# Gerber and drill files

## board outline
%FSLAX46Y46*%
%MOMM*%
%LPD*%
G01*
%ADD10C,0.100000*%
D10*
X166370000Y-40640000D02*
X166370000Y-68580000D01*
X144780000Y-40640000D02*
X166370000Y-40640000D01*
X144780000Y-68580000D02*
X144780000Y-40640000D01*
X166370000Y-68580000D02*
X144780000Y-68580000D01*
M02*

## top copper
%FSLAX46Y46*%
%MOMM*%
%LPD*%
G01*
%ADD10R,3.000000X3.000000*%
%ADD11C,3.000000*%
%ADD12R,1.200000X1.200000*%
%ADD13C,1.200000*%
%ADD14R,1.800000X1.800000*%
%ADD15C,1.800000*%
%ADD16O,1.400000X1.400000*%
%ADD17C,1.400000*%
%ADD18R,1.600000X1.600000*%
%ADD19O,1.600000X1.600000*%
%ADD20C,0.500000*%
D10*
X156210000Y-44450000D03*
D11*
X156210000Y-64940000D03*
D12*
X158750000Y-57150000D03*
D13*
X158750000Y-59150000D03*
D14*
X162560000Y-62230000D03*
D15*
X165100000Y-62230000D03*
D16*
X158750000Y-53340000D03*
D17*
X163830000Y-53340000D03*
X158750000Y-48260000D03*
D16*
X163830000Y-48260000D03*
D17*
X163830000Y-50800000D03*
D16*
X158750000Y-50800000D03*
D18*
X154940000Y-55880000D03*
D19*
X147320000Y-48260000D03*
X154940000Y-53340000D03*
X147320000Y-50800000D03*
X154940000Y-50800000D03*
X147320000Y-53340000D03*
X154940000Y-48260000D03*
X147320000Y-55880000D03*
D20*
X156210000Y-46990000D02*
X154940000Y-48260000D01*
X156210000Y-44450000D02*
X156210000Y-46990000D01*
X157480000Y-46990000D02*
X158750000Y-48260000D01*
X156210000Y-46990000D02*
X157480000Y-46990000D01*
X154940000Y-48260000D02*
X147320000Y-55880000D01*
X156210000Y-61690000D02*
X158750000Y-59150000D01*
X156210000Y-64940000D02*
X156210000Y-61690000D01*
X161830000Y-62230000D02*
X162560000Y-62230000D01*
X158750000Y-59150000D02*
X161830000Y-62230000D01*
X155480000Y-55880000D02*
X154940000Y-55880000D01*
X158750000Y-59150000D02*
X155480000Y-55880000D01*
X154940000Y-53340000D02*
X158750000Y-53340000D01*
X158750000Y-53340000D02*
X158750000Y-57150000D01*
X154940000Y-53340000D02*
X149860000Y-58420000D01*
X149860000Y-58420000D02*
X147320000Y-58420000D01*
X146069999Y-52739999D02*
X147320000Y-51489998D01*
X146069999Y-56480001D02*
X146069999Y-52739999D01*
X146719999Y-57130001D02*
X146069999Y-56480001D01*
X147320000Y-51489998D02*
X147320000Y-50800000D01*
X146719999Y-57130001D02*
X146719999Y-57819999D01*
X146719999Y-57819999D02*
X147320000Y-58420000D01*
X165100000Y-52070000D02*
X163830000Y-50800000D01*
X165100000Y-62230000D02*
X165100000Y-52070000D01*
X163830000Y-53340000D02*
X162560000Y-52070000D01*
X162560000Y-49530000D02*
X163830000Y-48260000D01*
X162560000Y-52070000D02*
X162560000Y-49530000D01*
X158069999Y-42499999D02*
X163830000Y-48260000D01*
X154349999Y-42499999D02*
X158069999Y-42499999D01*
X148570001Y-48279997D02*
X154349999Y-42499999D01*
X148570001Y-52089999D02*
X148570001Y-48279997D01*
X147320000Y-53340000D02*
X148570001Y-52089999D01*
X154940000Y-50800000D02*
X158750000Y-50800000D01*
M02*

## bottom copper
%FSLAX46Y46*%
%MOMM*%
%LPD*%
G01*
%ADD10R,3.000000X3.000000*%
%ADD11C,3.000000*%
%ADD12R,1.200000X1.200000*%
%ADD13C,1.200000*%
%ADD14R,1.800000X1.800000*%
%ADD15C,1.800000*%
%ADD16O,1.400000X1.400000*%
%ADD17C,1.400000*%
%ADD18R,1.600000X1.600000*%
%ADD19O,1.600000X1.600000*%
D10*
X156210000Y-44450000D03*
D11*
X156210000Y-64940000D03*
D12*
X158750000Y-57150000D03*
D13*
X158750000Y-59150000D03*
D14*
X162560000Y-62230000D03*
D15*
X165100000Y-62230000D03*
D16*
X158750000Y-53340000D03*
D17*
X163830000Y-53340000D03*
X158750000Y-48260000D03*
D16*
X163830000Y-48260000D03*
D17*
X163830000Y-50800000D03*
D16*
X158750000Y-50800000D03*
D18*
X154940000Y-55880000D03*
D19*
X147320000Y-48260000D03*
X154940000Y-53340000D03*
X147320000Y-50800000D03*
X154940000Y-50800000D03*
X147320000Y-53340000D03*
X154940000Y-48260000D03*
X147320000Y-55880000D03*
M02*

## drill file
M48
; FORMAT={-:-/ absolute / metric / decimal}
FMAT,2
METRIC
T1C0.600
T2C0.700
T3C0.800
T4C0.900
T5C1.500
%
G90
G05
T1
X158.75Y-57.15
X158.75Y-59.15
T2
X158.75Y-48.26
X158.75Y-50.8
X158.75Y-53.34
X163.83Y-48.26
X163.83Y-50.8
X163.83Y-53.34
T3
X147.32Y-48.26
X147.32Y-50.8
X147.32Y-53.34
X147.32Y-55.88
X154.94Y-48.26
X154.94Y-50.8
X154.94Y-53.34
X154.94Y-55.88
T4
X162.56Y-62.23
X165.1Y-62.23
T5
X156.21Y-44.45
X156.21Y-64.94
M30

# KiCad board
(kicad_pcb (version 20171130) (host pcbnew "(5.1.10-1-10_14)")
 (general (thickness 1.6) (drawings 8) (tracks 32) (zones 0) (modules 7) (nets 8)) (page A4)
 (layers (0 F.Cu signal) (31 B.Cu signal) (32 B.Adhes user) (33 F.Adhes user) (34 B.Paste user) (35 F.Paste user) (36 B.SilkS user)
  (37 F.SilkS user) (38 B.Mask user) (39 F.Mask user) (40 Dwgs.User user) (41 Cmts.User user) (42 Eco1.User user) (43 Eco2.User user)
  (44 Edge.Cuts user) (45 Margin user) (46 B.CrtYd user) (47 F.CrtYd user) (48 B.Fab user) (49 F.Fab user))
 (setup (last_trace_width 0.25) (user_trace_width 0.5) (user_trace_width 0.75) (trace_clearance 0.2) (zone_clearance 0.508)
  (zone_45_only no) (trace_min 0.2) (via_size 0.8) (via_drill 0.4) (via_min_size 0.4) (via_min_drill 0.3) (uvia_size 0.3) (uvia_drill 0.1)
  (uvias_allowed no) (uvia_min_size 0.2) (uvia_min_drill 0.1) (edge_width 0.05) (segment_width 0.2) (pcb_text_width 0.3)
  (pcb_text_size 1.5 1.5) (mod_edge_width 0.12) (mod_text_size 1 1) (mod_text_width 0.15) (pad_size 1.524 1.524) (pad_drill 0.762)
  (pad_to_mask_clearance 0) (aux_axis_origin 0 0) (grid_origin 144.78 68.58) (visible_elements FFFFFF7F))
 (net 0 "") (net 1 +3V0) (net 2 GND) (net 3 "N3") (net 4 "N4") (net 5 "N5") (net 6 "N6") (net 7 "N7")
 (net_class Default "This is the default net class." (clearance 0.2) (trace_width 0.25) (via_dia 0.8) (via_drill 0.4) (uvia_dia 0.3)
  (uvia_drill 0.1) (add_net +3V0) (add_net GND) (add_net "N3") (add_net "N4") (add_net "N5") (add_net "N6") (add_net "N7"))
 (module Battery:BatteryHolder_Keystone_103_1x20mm (layer B.Cu) (at 156.21 44.45 270)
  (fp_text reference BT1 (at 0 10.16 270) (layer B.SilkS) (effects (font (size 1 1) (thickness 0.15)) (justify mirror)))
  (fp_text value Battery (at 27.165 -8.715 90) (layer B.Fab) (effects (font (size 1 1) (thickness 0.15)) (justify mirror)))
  (pad 1 thru_hole rect (at 0 0 270) (size 3 3) (drill 1.5) (layers *.Cu *.Mask) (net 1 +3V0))
  (pad 2 thru_hole circle (at 20.49 0 270) (size 3 3) (drill 1.5) (layers *.Cu *.Mask) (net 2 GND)))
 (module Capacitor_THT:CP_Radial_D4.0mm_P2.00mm (layer F.Cu) (at 158.75 57.15 270)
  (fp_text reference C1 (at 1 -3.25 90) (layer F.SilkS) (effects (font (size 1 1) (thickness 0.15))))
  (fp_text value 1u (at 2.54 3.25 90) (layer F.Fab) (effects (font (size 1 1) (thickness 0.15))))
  (pad 1 thru_hole rect (at 0 0 270) (size 1.2 1.2) (drill 0.6) (layers *.Cu *.Mask) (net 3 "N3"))
  (pad 2 thru_hole circle (at 2 0 270) (size 1.2 1.2) (drill 0.6) (layers *.Cu *.Mask) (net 2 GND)))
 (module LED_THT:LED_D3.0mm (layer F.Cu) (at 162.56 62.23)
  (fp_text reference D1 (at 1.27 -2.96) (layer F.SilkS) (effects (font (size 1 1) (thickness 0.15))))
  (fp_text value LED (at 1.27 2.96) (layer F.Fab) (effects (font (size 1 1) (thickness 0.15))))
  (pad 1 thru_hole rect (at 0 0) (size 1.8 1.8) (drill 0.9) (layers *.Cu *.Mask) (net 2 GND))
  (pad 2 thru_hole circle (at 2.54 0) (size 1.8 1.8) (drill 0.9) (layers *.Cu *.Mask) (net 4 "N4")))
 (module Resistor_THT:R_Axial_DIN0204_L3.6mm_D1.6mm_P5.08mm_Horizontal (layer F.Cu) (at 163.83 53.34 180)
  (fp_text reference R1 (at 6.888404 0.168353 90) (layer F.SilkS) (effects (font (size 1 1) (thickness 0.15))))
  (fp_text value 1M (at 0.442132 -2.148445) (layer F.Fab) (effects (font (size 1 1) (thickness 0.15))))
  (pad 2 thru_hole oval (at 5.08 0 180) (size 1.4 1.4) (drill 0.7) (layers *.Cu *.Mask) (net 3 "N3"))
  (pad 1 thru_hole circle (at 0 0 180) (size 1.4 1.4) (drill 0.7) (layers *.Cu *.Mask) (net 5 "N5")))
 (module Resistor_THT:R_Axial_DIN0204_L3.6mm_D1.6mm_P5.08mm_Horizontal (layer F.Cu) (at 158.75 48.26)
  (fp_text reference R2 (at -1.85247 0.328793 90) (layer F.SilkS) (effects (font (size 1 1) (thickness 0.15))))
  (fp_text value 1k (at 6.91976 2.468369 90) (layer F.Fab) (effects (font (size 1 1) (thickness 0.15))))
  (pad 1 thru_hole circle (at 0 0) (size 1.4 1.4) (drill 0.7) (layers *.Cu *.Mask) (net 1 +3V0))
  (pad 2 thru_hole oval (at 5.08 0) (size 1.4 1.4) (drill 0.7) (layers *.Cu *.Mask) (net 5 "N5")))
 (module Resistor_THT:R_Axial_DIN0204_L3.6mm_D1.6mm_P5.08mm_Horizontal (layer F.Cu) (at 163.83 50.8 180)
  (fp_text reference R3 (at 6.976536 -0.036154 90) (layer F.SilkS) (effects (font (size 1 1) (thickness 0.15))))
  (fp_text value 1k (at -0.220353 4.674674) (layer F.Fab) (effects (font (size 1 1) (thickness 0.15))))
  (pad 1 thru_hole circle (at 0 0 180) (size 1.4 1.4) (drill 0.7) (layers *.Cu *.Mask) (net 4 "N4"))
  (pad 2 thru_hole oval (at 5.08 0 180) (size 1.4 1.4) (drill 0.7) (layers *.Cu *.Mask) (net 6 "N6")))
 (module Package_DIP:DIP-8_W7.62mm (layer F.Cu) (at 154.94 55.88 180)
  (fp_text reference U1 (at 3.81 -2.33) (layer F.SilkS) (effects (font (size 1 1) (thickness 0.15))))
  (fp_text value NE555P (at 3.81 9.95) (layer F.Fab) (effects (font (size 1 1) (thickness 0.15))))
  (pad 1 thru_hole rect (at 0 0 180) (size 1.6 1.6) (drill 0.8) (layers *.Cu *.Mask) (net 2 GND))
  (pad 5 thru_hole oval (at 7.62 7.62 180) (size 1.6 1.6) (drill 0.8) (layers *.Cu *.Mask) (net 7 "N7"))
  (pad 2 thru_hole oval (at 0 2.54 180) (size 1.6 1.6) (drill 0.8) (layers *.Cu *.Mask) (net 3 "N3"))
  (pad 6 thru_hole oval (at 7.62 5.08 180) (size 1.6 1.6) (drill 0.8) (layers *.Cu *.Mask) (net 3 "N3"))
  (pad 3 thru_hole oval (at 0 5.08 180) (size 1.6 1.6) (drill 0.8) (layers *.Cu *.Mask) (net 6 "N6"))
  (pad 7 thru_hole oval (at 7.62 2.54 180) (size 1.6 1.6) (drill 0.8) (layers *.Cu *.Mask) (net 5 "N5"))
  (pad 4 thru_hole oval (at 0 7.62 180) (size 1.6 1.6) (drill 0.8) (layers *.Cu *.Mask) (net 1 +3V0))
  (pad 8 thru_hole oval (at 7.62 0 180) (size 1.6 1.6) (drill 0.8) (layers *.Cu *.Mask) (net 1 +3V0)))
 (gr_line (start 166.37 40.64) (end 166.37 68.58) (layer Edge.Cuts) (width 0.1))
 (gr_line (start 144.78 40.64) (end 166.37 40.64) (layer Edge.Cuts) (width 0.1))
 (gr_line (start 144.78 68.58) (end 144.78 40.64) (layer Edge.Cuts) (width 0.1))
 (gr_line (start 166.37 68.58) (end 144.78 68.58) (layer Edge.Cuts) (width 0.1))
 (segment (start 156.21 46.99) (end 154.94 48.26) (width 0.5) (layer F.Cu) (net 1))
 (segment (start 156.21 44.45) (end 156.21 46.99) (width 0.5) (layer F.Cu) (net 1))
 (segment (start 157.48 46.99) (end 158.75 48.26) (width 0.5) (layer F.Cu) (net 1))
 (segment (start 156.21 46.99) (end 157.48 46.99) (width 0.5) (layer F.Cu) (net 1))
 (segment (start 154.94 48.26) (end 147.32 55.88) (width 0.5) (layer F.Cu) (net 1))
 (segment (start 156.21 61.69) (end 158.75 59.15) (width 0.5) (layer F.Cu) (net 2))
 (segment (start 156.21 64.94) (end 156.21 61.69) (width 0.5) (layer F.Cu) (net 2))
 (segment (start 161.83 62.23) (end 162.56 62.23) (width 0.5) (layer F.Cu) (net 2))
 (segment (start 158.75 59.15) (end 161.83 62.23) (width 0.5) (layer F.Cu) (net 2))
 (segment (start 155.48 55.88) (end 154.94 55.88) (width 0.5) (layer F.Cu) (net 2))
 (segment (start 158.75 59.15) (end 155.48 55.88) (width 0.5) (layer F.Cu) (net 2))
 (segment (start 154.94 53.34) (end 158.75 53.34) (width 0.5) (layer F.Cu) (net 3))
 (segment (start 158.75 53.34) (end 158.75 57.15) (width 0.5) (layer F.Cu) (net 3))
 (segment (start 154.94 53.34) (end 149.86 58.42) (width 0.5) (layer F.Cu) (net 3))
 (segment (start 149.86 58.42) (end 147.32 58.42) (width 0.5) (layer F.Cu) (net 3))
 (segment (start 146.069999 52.739999) (end 147.32 51.489998) (width 0.5) (layer F.Cu) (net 3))
 (segment (start 146.069999 56.480001) (end 146.069999 52.739999) (width 0.5) (layer F.Cu) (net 3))
 (segment (start 146.719999 57.130001) (end 146.069999 56.480001) (width 0.5) (layer F.Cu) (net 3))
 (segment (start 147.32 51.489998) (end 147.32 50.8) (width 0.5) (layer F.Cu) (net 3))
 (segment (start 146.719999 57.130001) (end 146.719999 57.819999) (width 0.5) (layer F.Cu) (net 3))
 (segment (start 146.719999 57.819999) (end 147.32 58.42) (width 0.5) (layer F.Cu) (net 3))
 (segment (start 165.1 52.07) (end 163.83 50.8) (width 0.5) (layer F.Cu) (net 4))
 (segment (start 165.1 62.23) (end 165.1 52.07) (width 0.5) (layer F.Cu) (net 4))
 (segment (start 163.83 53.34) (end 162.56 52.07) (width 0.5) (layer F.Cu) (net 5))
 (segment (start 162.56 49.53) (end 163.83 48.26) (width 0.5) (layer F.Cu) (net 5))
 (segment (start 162.56 52.07) (end 162.56 49.53) (width 0.5) (layer F.Cu) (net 5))
 (segment (start 158.069999 42.499999) (end 163.83 48.26) (width 0.5) (layer F.Cu) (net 5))
 (segment (start 154.349999 42.499999) (end 158.069999 42.499999) (width 0.5) (layer F.Cu) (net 5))
 (segment (start 148.570001 48.279997) (end 154.349999 42.499999) (width 0.5) (layer F.Cu) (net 5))
 (segment (start 148.570001 52.089999) (end 148.570001 48.279997) (width 0.5) (layer F.Cu) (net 5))
 (segment (start 147.32 53.34) (end 148.570001 52.089999) (width 0.5) (layer F.Cu) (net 5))
 (segment (start 154.94 50.8) (end 158.75 50.8) (width 0.5) (layer F.Cu) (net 6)))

